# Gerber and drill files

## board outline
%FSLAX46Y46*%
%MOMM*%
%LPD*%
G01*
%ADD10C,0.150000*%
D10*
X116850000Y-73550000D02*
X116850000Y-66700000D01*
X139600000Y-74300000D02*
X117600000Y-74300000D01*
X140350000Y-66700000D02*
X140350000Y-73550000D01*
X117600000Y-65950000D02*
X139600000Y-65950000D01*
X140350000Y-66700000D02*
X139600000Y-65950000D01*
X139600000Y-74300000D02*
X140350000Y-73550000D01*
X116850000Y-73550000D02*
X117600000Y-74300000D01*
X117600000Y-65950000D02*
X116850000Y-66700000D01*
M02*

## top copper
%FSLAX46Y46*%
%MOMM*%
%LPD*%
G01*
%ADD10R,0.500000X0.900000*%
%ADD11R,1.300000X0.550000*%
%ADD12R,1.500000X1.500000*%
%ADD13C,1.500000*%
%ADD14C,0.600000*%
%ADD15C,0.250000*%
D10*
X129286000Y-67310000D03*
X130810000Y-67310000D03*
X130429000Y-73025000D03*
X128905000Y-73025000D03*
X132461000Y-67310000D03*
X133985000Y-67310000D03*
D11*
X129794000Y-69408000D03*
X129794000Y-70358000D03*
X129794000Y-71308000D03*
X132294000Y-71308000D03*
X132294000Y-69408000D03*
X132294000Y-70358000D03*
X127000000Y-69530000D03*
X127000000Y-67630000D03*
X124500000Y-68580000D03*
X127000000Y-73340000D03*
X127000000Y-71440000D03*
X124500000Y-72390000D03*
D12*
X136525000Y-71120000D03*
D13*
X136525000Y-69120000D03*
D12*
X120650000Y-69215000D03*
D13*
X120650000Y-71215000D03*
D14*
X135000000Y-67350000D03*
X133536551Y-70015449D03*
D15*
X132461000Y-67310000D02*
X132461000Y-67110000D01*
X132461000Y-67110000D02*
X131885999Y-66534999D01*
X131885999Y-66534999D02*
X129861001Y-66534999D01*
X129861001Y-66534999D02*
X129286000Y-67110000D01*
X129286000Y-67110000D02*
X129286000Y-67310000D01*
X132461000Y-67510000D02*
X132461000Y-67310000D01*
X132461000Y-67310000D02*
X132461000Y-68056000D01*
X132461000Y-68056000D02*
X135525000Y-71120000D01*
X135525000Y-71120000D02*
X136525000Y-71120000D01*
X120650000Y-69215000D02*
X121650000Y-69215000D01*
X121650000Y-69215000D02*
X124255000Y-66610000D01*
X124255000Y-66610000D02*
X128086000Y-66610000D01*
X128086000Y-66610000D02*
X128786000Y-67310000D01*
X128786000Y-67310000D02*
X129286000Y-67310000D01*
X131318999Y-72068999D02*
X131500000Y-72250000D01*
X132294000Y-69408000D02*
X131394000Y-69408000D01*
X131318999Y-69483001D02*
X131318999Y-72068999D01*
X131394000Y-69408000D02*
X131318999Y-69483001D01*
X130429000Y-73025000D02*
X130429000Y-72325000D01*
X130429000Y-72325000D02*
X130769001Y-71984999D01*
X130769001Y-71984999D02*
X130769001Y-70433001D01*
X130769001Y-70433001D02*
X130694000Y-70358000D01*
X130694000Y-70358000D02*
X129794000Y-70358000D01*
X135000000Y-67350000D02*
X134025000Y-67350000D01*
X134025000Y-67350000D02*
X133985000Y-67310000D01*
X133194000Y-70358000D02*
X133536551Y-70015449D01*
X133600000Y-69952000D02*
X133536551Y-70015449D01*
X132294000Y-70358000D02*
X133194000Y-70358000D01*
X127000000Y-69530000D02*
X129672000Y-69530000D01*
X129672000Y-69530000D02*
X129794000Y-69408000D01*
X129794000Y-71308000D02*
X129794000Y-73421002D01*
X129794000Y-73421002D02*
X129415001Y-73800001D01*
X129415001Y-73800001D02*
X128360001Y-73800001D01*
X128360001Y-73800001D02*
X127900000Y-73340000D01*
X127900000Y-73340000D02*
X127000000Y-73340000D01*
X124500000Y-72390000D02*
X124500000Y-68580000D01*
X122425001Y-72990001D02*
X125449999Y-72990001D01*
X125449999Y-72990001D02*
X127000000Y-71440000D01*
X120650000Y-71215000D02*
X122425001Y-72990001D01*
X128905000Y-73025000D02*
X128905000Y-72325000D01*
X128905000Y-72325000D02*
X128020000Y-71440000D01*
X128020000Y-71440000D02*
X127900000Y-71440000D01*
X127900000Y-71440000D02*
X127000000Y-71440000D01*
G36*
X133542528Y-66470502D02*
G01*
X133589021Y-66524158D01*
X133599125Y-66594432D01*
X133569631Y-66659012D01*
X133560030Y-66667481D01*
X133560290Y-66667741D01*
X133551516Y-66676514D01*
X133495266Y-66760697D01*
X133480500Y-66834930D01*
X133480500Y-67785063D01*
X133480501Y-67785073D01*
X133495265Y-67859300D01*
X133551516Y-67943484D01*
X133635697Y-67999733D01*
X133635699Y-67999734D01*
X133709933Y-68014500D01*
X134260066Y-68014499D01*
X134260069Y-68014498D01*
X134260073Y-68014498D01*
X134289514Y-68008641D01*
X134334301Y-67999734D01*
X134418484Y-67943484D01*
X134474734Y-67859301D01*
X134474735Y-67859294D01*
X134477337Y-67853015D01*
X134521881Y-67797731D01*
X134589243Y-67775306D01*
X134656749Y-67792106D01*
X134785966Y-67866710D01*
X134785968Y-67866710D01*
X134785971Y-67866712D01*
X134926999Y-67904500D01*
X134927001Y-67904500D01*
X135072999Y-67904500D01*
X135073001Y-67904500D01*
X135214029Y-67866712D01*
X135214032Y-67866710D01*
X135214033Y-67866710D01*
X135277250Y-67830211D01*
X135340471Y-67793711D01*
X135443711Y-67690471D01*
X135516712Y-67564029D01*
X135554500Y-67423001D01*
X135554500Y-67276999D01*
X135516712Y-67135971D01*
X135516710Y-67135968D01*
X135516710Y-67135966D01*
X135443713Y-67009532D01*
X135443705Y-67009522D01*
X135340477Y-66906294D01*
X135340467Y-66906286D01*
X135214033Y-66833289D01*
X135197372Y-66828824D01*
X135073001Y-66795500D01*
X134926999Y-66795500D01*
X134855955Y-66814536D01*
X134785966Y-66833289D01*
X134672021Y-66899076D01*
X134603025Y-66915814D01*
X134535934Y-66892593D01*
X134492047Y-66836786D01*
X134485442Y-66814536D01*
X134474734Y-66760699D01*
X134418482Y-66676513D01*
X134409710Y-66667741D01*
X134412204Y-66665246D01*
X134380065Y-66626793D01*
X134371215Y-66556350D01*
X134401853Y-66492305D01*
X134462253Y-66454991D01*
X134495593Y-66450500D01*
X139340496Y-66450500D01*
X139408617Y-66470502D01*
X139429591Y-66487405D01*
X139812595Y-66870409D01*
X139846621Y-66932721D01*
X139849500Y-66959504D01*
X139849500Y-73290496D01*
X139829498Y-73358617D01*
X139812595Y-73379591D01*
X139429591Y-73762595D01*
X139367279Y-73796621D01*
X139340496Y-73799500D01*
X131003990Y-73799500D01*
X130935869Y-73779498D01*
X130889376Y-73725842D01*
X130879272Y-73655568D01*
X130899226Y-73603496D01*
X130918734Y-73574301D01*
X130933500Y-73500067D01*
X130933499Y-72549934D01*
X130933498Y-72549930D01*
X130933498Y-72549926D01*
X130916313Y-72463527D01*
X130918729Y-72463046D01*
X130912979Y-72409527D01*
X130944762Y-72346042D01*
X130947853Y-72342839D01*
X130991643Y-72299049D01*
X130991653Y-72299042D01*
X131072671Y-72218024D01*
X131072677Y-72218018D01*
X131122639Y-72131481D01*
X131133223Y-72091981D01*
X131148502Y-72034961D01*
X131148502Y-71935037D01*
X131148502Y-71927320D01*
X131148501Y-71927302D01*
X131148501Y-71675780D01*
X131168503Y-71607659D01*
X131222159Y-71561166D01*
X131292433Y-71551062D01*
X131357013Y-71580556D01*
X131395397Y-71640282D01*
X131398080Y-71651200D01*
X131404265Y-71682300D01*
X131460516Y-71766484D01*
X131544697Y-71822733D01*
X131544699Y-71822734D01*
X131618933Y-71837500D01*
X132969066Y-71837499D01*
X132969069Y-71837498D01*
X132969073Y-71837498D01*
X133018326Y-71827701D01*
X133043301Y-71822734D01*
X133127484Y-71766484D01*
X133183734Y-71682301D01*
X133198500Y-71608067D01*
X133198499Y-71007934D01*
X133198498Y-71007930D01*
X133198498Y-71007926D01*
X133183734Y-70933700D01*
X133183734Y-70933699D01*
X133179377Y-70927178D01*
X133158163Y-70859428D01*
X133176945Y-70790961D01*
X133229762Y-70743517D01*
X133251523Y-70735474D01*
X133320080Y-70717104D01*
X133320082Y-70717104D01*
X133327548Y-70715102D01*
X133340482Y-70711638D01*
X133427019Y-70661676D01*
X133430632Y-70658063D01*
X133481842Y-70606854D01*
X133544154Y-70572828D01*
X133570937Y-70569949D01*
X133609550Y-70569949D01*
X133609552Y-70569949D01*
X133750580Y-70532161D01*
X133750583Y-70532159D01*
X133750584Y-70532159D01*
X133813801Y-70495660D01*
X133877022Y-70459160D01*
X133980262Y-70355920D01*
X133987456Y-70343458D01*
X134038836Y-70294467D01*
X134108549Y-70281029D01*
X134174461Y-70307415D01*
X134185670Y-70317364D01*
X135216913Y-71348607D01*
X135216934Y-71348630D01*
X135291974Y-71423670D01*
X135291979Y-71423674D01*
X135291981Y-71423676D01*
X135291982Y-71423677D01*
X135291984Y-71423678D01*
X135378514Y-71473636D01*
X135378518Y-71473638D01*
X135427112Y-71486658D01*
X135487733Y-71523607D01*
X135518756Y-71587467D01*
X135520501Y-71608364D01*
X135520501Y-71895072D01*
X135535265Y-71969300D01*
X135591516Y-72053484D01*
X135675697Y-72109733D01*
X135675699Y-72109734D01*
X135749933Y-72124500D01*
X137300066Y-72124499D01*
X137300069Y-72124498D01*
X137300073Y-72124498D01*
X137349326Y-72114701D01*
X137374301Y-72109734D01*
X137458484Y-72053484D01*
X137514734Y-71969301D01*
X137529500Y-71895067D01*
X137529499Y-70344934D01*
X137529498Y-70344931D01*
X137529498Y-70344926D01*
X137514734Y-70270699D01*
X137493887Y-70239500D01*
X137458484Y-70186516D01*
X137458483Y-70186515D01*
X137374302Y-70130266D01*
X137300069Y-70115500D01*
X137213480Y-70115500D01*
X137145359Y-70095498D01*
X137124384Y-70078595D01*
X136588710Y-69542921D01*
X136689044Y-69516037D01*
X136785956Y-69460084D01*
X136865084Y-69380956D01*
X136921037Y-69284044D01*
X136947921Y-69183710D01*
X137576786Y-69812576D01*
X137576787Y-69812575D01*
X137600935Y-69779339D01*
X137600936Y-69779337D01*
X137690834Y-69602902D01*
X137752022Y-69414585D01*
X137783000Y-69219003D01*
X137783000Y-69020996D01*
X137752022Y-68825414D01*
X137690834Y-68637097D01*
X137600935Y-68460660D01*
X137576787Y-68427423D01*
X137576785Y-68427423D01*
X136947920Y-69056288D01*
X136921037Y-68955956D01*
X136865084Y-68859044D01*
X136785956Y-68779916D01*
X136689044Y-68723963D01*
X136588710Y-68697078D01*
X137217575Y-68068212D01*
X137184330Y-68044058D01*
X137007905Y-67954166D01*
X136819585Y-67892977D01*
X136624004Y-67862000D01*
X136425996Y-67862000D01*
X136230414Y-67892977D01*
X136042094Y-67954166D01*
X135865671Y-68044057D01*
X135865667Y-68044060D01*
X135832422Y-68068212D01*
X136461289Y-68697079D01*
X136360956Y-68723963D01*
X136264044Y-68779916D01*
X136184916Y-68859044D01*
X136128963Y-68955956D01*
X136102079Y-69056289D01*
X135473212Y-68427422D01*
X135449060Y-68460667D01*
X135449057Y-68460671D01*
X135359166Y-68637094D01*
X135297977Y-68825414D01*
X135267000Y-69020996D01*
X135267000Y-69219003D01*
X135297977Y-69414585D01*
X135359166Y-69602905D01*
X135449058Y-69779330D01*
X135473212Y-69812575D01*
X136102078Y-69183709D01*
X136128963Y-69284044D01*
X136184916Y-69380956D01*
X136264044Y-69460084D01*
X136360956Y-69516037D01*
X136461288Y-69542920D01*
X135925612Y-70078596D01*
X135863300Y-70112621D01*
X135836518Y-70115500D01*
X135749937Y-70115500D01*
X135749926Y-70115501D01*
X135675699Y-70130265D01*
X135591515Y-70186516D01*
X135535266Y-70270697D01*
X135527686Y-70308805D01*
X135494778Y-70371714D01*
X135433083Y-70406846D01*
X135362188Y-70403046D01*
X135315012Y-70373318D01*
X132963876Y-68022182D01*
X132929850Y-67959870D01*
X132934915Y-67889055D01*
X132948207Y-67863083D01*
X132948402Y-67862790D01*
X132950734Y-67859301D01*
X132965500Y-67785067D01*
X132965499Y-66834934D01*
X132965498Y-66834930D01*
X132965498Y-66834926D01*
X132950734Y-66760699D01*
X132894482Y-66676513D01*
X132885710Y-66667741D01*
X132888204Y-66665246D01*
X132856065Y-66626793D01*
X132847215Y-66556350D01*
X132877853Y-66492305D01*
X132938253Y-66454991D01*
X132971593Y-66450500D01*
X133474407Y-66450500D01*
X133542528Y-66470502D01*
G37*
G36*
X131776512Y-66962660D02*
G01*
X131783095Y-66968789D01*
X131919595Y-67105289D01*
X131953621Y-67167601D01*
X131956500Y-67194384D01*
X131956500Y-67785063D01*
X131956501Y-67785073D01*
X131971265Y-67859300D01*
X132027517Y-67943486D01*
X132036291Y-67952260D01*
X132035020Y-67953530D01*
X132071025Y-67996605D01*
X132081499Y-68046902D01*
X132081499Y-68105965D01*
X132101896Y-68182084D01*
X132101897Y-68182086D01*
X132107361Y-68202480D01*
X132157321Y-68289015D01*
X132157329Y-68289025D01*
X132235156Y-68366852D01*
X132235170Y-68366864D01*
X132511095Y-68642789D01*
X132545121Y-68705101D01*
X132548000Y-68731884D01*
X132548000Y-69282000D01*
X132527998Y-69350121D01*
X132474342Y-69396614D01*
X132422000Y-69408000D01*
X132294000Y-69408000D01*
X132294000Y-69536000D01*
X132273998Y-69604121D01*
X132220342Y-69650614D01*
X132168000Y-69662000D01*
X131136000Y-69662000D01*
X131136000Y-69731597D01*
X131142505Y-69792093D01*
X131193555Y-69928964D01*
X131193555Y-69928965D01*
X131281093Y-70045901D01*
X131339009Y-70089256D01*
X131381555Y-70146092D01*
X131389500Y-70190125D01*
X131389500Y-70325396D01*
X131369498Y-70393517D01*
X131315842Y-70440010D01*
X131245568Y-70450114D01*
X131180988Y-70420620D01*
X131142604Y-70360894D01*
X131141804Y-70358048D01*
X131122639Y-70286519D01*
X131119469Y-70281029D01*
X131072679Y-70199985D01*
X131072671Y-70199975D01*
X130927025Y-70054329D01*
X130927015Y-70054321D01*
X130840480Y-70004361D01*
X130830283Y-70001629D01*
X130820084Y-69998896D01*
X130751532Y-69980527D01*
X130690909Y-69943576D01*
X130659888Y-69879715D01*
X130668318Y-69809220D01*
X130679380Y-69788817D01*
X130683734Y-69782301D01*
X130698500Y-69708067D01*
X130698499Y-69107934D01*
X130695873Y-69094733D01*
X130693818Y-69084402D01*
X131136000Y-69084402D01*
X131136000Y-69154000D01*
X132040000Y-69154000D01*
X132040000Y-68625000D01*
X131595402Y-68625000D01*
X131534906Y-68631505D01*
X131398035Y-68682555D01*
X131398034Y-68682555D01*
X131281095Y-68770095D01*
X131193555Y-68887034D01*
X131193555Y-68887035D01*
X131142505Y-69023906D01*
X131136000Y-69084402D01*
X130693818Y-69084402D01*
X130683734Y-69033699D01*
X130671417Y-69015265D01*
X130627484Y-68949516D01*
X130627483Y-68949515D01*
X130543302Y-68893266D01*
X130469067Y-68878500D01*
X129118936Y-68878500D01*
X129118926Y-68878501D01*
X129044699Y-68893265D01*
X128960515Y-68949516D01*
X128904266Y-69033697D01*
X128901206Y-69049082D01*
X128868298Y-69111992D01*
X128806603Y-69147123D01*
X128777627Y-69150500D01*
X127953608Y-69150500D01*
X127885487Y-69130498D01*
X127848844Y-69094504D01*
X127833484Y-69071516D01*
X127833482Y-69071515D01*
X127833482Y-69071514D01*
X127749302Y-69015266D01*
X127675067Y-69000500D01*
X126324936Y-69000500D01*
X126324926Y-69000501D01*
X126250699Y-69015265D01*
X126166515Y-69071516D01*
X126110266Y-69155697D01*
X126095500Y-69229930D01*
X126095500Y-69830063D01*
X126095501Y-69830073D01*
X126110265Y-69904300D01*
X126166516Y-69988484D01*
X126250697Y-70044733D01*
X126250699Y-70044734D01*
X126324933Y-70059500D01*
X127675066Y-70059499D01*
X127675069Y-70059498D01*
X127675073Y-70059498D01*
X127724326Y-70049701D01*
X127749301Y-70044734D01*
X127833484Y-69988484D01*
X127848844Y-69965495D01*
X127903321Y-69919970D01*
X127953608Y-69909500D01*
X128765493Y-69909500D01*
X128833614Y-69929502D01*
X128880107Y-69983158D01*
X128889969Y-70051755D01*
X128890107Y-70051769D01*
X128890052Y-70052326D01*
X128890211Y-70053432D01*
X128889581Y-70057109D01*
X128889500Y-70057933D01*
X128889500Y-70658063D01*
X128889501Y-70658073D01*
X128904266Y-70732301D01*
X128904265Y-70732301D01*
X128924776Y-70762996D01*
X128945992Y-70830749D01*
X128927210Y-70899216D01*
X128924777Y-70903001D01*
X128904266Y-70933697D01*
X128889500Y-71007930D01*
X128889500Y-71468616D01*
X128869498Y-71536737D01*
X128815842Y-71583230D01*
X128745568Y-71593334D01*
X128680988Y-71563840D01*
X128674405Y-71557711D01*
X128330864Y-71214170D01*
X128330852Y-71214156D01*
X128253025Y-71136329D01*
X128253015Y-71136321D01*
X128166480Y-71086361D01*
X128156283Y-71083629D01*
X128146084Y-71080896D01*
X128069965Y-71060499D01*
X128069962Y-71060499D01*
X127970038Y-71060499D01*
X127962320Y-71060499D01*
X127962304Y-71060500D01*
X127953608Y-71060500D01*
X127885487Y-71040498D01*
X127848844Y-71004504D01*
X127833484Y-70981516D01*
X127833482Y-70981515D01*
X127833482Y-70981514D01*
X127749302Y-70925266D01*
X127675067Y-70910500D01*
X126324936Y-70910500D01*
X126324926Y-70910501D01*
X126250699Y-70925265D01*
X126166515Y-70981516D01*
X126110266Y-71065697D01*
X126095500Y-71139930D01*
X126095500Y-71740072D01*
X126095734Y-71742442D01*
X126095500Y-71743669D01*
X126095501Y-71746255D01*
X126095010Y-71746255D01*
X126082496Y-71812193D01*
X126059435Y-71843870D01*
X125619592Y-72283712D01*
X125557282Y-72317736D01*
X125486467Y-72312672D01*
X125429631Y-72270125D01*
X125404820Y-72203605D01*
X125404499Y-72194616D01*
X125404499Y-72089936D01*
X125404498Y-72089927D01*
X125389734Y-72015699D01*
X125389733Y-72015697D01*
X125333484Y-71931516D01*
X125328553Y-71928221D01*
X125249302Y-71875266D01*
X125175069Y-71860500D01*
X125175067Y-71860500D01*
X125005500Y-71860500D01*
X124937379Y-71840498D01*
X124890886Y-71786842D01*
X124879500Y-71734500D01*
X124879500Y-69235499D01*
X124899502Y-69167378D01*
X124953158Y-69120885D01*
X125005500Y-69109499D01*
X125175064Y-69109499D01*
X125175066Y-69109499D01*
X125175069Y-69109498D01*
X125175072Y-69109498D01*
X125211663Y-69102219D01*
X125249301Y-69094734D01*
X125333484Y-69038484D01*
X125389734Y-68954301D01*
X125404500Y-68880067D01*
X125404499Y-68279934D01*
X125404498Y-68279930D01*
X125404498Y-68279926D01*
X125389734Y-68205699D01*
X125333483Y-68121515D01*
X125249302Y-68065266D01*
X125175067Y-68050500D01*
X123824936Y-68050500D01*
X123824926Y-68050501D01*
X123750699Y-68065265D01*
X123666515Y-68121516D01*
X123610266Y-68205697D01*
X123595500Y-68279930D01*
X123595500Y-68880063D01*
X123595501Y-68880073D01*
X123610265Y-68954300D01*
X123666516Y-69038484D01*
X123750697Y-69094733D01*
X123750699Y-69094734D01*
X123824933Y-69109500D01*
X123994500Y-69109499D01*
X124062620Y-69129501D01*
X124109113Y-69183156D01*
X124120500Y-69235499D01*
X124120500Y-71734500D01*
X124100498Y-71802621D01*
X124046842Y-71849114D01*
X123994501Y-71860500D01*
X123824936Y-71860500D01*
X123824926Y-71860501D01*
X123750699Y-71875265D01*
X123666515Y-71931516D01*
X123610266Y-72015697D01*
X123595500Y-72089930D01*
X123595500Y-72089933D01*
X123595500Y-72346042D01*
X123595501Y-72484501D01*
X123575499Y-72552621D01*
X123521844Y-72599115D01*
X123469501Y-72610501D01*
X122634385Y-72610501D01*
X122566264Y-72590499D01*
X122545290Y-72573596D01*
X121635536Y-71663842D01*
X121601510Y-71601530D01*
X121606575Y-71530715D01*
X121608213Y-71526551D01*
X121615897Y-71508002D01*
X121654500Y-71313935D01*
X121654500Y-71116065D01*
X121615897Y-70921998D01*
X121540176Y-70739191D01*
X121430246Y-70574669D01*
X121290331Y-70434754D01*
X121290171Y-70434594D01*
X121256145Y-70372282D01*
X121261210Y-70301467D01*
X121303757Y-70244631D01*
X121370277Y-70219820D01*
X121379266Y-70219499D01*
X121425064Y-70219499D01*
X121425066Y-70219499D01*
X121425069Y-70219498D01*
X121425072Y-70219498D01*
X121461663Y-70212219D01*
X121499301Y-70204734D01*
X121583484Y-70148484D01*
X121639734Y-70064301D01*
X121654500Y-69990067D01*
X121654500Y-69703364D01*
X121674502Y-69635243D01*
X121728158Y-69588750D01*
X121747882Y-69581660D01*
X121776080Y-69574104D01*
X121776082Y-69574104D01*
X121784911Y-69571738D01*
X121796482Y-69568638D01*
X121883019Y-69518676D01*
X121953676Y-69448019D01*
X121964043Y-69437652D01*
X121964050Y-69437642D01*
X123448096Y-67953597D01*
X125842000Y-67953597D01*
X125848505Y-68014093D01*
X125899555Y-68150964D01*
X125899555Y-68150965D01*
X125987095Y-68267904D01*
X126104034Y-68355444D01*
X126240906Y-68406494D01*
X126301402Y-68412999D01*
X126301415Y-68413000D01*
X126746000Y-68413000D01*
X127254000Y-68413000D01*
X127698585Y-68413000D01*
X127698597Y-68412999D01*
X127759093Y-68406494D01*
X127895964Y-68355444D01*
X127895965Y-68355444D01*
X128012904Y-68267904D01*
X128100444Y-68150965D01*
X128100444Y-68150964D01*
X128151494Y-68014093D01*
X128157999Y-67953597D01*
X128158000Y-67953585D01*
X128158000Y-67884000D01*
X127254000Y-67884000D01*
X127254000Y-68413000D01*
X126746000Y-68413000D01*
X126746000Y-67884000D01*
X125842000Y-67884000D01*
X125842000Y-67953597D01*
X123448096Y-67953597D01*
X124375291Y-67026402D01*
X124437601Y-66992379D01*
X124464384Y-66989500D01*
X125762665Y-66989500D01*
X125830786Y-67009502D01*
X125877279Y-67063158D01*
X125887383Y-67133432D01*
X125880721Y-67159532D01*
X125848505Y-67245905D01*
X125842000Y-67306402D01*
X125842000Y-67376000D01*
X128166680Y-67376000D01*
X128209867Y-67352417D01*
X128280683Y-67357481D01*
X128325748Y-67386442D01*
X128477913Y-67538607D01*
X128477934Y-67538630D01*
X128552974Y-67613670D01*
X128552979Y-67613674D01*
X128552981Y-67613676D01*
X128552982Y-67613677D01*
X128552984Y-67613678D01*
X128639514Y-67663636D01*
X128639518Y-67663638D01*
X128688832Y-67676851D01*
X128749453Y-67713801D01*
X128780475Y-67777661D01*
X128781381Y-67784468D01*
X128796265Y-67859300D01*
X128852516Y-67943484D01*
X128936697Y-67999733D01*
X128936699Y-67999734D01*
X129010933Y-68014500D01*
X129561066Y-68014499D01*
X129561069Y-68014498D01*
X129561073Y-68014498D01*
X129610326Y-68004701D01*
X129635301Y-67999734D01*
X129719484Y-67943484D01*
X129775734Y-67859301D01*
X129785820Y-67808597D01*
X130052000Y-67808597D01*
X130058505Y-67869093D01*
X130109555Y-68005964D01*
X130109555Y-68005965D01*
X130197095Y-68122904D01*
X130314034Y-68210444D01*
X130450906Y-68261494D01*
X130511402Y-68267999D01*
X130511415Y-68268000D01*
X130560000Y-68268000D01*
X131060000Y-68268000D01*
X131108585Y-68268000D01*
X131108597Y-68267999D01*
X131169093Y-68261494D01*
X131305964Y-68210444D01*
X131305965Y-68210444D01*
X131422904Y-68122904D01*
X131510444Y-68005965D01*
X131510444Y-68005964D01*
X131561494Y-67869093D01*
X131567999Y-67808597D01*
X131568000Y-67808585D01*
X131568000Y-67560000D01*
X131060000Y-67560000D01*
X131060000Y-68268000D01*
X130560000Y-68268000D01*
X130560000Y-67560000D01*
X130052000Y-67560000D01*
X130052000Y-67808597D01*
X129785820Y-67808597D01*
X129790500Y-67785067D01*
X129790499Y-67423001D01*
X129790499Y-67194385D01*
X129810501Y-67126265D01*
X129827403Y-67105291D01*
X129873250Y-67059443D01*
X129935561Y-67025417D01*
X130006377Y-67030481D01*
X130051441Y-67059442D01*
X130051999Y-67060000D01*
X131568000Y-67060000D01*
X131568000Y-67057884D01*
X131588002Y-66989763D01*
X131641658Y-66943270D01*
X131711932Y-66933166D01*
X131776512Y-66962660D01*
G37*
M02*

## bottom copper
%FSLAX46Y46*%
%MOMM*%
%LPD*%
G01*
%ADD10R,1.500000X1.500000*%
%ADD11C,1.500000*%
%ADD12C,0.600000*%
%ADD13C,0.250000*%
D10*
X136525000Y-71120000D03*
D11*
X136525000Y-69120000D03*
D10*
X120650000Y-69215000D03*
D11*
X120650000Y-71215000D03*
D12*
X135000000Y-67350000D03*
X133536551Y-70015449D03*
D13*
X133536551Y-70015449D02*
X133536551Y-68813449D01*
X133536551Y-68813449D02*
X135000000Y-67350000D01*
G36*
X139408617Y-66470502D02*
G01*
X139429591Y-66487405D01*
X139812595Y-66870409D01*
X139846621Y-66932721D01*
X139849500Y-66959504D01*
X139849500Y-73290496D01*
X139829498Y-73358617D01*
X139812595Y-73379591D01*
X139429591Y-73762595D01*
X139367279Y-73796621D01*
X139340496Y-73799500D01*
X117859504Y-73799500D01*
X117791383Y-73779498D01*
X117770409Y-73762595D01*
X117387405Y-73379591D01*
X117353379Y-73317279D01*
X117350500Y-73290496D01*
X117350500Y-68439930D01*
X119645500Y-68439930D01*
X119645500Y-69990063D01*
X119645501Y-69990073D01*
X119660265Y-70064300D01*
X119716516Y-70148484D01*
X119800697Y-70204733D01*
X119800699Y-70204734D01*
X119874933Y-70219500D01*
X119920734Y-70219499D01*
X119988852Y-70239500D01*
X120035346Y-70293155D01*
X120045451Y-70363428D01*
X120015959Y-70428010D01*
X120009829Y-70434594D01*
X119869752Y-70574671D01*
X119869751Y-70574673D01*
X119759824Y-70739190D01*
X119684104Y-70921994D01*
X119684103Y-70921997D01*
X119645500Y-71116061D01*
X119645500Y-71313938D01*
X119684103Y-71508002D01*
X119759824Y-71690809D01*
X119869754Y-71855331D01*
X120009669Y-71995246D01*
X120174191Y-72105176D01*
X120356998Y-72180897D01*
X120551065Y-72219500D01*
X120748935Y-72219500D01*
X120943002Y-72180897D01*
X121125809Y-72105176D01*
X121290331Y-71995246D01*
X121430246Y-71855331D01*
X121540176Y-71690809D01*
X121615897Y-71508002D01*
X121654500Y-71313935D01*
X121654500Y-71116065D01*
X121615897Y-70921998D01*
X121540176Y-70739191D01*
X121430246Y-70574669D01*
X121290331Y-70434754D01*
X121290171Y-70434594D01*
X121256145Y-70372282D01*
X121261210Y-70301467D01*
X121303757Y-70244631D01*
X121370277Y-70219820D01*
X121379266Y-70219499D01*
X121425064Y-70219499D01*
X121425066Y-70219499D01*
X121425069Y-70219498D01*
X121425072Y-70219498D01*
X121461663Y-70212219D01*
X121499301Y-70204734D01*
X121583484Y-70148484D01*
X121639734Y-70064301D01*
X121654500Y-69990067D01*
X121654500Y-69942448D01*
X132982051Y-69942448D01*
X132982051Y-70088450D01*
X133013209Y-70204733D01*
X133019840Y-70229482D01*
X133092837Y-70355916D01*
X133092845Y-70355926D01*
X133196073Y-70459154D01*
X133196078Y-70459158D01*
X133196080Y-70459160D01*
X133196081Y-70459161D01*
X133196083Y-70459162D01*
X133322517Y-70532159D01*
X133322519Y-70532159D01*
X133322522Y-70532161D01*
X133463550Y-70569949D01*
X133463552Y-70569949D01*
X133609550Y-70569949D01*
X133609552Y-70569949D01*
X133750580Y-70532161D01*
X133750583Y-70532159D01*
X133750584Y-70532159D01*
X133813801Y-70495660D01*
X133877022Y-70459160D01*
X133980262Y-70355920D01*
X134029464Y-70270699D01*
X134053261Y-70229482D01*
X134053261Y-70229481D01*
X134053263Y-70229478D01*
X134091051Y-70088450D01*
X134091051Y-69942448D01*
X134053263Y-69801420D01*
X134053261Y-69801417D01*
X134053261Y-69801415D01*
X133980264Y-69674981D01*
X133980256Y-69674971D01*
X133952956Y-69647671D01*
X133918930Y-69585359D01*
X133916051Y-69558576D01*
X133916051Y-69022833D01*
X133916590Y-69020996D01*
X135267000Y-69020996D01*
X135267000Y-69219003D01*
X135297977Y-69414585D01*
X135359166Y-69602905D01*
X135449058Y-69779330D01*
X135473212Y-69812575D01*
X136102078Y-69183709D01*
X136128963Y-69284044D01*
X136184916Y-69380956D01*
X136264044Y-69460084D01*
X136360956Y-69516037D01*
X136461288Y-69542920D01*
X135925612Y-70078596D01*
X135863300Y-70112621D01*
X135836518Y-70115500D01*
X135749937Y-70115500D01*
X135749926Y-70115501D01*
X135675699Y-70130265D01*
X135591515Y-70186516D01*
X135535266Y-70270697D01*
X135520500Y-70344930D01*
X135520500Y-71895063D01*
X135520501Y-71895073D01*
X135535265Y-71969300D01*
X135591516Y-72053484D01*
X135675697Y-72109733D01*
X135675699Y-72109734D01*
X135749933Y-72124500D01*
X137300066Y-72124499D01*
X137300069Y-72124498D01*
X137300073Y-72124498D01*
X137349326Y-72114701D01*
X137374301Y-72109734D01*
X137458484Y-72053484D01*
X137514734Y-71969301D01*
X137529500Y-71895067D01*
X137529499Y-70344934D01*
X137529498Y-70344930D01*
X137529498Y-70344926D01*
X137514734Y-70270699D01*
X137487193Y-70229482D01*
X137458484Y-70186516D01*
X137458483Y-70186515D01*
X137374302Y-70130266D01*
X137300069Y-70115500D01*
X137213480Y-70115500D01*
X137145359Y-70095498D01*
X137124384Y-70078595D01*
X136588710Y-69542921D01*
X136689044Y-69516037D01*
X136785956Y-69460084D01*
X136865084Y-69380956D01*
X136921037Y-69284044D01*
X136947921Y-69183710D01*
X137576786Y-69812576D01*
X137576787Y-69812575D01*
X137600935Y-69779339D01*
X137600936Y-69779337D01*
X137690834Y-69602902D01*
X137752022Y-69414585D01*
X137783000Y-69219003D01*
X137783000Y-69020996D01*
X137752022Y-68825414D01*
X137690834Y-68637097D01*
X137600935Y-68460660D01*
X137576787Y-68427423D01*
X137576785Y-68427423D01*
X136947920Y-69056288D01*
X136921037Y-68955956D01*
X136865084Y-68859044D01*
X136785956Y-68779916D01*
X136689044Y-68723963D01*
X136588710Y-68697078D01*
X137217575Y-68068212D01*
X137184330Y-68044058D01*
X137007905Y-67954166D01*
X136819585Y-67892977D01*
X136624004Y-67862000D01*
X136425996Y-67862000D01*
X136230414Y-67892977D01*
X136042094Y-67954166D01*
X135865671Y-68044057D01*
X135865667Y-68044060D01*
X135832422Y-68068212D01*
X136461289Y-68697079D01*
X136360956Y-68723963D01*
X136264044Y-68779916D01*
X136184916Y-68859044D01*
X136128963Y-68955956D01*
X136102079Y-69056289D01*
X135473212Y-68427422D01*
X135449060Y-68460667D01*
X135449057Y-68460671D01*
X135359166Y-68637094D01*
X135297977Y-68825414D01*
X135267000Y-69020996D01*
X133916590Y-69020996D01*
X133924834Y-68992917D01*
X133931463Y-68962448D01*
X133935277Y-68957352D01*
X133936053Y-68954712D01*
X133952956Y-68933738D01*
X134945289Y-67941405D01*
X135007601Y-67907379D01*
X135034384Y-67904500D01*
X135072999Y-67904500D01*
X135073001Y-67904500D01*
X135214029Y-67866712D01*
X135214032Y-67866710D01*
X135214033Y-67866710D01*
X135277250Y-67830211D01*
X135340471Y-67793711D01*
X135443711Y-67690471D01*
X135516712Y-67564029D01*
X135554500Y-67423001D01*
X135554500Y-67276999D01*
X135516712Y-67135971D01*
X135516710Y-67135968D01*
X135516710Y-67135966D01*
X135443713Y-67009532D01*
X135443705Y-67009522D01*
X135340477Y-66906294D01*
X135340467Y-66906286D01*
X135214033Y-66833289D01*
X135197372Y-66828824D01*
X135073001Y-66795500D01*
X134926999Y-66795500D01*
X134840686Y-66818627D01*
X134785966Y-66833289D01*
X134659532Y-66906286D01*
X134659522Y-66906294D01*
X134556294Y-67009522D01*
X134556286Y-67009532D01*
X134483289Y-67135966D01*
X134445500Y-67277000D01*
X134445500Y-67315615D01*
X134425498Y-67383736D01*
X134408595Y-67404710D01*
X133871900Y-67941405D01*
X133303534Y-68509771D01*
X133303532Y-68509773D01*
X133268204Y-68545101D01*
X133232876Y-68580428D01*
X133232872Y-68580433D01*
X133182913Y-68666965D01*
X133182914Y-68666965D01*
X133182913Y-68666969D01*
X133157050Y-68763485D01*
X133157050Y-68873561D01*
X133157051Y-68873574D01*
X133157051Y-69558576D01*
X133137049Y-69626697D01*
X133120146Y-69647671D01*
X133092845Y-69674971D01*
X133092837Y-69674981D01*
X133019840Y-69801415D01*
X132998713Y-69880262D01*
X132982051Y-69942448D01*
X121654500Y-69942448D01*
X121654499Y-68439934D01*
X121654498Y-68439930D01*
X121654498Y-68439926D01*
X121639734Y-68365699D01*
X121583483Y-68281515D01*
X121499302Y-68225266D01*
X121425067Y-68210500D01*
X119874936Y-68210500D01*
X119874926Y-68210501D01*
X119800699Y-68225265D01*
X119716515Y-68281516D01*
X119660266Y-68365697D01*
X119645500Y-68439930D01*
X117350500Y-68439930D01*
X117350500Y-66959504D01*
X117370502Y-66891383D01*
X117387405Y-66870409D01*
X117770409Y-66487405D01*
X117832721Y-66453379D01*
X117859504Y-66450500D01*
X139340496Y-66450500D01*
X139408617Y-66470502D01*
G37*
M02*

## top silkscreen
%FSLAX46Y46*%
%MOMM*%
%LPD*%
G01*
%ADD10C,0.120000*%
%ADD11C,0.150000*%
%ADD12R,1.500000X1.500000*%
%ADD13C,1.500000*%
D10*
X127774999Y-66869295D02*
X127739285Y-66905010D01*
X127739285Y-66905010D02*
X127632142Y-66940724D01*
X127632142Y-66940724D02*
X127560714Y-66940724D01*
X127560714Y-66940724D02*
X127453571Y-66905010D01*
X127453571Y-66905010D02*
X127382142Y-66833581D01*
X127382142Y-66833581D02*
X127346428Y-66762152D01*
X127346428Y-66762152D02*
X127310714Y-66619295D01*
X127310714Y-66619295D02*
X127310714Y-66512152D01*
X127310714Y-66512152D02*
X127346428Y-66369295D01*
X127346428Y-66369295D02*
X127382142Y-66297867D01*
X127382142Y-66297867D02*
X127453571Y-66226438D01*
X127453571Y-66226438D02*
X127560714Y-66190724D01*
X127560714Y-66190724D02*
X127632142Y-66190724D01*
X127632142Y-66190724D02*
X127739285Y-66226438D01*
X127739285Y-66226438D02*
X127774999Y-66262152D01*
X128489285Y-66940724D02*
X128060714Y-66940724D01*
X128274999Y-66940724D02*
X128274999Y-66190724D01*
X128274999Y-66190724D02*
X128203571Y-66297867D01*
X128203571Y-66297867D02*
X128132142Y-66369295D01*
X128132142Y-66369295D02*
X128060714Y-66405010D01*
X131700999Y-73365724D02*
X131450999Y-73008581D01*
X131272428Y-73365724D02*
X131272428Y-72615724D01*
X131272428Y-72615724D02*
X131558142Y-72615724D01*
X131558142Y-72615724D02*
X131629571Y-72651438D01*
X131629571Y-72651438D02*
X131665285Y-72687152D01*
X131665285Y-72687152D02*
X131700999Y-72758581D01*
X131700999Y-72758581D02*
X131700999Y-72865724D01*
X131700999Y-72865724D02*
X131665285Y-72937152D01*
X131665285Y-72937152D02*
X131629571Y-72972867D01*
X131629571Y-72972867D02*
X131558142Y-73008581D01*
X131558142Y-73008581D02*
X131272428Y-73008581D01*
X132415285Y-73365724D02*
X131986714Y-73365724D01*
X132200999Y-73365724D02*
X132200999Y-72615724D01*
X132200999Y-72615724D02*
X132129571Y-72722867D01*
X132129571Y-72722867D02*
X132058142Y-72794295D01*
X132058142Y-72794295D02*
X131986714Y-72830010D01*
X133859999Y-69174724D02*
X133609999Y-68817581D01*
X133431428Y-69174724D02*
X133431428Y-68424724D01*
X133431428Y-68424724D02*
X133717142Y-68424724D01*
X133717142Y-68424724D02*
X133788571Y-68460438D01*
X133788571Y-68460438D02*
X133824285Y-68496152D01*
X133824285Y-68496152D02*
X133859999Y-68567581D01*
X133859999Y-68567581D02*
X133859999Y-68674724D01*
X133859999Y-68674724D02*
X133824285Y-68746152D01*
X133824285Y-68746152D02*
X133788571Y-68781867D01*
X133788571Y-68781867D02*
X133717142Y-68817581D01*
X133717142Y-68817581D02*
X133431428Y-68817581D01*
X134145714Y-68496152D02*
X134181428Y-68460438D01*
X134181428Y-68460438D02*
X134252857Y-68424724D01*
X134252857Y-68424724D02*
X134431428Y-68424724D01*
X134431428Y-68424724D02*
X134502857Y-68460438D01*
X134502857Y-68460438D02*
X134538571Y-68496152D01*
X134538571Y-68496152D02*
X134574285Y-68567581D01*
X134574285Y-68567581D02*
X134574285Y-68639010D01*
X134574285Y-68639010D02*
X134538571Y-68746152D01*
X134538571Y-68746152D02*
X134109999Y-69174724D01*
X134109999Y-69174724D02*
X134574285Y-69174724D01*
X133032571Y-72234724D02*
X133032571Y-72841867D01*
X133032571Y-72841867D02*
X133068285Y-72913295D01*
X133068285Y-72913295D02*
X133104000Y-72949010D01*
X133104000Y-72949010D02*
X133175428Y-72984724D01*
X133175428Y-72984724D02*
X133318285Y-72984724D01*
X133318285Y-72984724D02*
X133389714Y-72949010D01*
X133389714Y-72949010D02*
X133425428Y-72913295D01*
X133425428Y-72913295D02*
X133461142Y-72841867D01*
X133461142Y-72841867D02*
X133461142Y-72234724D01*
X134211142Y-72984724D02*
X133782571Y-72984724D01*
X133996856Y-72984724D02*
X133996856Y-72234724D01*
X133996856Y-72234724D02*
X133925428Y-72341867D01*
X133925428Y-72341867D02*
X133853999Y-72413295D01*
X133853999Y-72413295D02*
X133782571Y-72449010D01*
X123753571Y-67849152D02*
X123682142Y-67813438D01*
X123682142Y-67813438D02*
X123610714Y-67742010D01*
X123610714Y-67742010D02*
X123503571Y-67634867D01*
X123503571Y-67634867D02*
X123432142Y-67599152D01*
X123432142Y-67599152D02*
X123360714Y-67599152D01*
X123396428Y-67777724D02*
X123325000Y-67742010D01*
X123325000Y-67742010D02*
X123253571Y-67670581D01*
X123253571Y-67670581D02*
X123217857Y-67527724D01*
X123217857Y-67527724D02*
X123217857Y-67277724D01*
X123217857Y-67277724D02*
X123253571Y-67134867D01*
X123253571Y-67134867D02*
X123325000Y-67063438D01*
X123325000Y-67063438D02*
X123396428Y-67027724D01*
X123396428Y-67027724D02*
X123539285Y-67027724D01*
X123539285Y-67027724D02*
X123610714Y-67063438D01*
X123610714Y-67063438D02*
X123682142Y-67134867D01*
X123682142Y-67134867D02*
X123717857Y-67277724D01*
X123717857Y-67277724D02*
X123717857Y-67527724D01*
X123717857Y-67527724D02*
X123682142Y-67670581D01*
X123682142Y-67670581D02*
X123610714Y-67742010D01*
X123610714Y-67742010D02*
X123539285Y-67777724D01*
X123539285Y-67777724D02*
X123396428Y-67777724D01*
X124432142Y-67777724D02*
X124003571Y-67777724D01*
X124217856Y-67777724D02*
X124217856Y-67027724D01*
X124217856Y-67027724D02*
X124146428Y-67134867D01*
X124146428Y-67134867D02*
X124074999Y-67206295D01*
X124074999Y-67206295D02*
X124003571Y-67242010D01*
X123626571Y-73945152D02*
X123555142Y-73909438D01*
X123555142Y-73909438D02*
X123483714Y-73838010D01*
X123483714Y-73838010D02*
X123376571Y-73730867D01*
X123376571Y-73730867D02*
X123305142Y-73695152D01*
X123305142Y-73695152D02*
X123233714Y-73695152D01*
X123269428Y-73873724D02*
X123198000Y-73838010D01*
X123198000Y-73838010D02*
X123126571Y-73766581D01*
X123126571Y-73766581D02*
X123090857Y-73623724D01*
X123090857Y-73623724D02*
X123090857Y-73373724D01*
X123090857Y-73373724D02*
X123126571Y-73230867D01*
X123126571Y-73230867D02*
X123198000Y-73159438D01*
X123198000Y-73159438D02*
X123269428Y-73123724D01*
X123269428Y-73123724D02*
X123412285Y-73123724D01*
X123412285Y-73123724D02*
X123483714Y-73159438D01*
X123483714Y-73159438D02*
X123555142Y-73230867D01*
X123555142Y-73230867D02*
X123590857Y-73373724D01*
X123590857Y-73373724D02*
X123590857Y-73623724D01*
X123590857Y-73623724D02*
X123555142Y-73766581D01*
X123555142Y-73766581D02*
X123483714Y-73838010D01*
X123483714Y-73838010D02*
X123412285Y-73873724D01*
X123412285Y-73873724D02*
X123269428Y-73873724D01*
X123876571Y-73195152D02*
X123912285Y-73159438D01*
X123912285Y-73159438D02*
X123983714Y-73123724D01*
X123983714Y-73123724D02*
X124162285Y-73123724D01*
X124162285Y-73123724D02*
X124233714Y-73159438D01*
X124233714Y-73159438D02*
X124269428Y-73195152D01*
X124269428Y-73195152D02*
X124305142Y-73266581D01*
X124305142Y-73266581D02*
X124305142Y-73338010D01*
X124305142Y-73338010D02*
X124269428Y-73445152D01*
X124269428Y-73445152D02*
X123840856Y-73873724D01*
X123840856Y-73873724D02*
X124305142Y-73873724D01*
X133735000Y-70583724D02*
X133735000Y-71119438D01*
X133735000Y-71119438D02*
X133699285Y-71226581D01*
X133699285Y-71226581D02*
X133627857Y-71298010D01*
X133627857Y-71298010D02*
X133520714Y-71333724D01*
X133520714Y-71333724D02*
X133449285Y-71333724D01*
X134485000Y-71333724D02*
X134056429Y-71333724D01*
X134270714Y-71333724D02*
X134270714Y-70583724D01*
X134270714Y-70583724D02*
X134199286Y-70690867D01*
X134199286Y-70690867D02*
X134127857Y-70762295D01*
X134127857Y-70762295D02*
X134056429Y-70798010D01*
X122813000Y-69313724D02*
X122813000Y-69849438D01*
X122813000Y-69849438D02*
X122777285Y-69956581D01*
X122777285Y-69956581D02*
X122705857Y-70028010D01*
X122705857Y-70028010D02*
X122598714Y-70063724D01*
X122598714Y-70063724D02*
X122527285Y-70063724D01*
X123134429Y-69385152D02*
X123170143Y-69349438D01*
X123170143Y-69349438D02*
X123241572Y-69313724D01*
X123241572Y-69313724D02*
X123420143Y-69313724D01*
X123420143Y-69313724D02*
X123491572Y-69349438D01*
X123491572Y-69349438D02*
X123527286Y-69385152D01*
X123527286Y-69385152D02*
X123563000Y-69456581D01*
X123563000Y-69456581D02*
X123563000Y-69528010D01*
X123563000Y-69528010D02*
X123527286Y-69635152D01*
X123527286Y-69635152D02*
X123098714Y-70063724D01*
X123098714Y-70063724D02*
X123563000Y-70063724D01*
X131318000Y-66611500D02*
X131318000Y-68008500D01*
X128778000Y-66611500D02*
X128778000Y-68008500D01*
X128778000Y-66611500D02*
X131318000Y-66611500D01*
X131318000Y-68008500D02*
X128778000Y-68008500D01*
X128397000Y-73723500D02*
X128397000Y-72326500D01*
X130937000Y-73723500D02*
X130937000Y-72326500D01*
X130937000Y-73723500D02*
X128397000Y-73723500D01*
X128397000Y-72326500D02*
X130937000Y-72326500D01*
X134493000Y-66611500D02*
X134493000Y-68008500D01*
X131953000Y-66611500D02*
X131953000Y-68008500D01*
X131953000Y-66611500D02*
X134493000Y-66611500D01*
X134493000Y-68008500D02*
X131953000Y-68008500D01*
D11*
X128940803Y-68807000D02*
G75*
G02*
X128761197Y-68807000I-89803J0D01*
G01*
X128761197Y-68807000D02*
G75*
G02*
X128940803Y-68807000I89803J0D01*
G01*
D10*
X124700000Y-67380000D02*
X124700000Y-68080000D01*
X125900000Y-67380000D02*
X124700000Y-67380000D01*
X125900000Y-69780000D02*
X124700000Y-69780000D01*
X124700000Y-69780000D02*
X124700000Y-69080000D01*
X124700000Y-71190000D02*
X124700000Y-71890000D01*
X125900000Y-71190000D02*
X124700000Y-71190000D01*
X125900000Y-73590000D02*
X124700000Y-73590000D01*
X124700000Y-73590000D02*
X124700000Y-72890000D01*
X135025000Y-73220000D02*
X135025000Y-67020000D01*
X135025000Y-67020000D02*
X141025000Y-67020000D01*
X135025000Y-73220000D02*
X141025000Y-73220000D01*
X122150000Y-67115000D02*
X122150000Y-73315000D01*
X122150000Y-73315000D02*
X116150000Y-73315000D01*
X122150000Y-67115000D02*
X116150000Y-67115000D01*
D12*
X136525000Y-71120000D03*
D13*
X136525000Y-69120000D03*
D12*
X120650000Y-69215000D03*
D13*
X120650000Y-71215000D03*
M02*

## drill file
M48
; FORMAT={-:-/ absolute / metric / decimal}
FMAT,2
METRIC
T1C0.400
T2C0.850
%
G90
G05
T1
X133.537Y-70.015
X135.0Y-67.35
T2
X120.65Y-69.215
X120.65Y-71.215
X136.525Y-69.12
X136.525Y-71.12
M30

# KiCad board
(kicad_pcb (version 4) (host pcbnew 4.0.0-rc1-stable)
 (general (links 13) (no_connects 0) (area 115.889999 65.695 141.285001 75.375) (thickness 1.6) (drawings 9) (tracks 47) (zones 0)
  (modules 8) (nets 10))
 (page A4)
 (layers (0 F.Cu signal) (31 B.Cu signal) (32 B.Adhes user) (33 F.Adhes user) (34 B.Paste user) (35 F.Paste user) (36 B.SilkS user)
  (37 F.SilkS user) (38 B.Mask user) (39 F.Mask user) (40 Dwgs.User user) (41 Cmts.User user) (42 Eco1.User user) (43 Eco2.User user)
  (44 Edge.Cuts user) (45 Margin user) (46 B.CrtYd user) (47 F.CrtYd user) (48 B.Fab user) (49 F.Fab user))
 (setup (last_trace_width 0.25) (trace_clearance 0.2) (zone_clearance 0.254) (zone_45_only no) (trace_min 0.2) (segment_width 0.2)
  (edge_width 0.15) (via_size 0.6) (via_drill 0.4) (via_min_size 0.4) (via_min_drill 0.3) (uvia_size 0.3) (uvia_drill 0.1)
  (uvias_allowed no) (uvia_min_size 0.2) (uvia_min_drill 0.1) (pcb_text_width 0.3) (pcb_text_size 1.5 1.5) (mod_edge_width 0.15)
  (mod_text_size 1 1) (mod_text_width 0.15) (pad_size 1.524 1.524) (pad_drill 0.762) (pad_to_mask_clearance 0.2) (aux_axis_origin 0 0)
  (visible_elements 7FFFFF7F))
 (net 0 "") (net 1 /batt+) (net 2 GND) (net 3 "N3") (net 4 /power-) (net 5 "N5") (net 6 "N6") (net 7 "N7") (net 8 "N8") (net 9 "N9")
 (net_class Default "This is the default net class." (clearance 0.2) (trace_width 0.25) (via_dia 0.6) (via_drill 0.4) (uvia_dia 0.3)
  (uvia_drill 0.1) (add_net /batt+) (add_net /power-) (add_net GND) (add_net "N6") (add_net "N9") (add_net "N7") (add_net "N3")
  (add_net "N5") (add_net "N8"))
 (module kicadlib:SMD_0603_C (layer F.Cu) (at 130.81 67.31)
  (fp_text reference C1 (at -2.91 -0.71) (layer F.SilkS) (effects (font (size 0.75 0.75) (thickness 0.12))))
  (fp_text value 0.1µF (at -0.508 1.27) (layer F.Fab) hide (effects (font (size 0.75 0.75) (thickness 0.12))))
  (fp_line (start 0.508 -0.6985) (end 0.508 0.6985) (layer F.SilkS) (width 0.12))
  (fp_line (start -2.032 -0.6985) (end -2.032 0.6985) (layer F.SilkS) (width 0.12))
  (fp_line (start -2.032 -0.6985) (end 0.508 -0.6985) (layer F.SilkS) (width 0.12))
  (fp_line (start 0.508 0.6985) (end -2.032 0.6985) (layer F.SilkS) (width 0.12))
  (pad 1 smd rect (at -1.524 0) (size 0.5 0.9) (layers F.Cu F.Paste F.Mask) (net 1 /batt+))
  (pad 2 smd rect (at 0 0) (size 0.5 0.9) (layers F.Cu F.Paste F.Mask) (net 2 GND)))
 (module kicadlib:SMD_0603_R (layer F.Cu) (at 128.905 73.025 180)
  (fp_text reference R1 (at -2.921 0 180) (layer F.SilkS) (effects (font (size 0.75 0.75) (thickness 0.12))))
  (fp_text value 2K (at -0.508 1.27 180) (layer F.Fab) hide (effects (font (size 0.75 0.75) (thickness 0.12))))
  (fp_line (start 0.508 -0.6985) (end 0.508 0.6985) (layer F.SilkS) (width 0.12))
  (fp_line (start -2.032 -0.6985) (end -2.032 0.6985) (layer F.SilkS) (width 0.12))
  (fp_line (start -2.032 -0.6985) (end 0.508 -0.6985) (layer F.SilkS) (width 0.12))
  (fp_line (start 0.508 0.6985) (end -2.032 0.6985) (layer F.SilkS) (width 0.12))
  (pad 1 smd rect (at -1.524 0 180) (size 0.5 0.9) (layers F.Cu F.Paste F.Mask) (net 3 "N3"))
  (pad 2 smd rect (at 0 0 180) (size 0.5 0.9) (layers F.Cu F.Paste F.Mask) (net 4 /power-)))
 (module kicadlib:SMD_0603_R (layer F.Cu) (at 133.985 67.31)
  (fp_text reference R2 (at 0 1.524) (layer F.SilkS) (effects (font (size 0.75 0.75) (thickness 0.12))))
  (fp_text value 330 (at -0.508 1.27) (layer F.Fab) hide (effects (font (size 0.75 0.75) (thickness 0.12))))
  (fp_line (start 0.508 -0.6985) (end 0.508 0.6985) (layer F.SilkS) (width 0.12))
  (fp_line (start -2.032 -0.6985) (end -2.032 0.6985) (layer F.SilkS) (width 0.12))
  (fp_line (start -2.032 -0.6985) (end 0.508 -0.6985) (layer F.SilkS) (width 0.12))
  (fp_line (start 0.508 0.6985) (end -2.032 0.6985) (layer F.SilkS) (width 0.12))
  (pad 1 smd rect (at -1.524 0) (size 0.5 0.9) (layers F.Cu F.Paste F.Mask) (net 1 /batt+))
  (pad 2 smd rect (at 0 0) (size 0.5 0.9) (layers F.Cu F.Paste F.Mask) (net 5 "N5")))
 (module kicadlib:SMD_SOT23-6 (layer F.Cu) (at 129.794 70.358)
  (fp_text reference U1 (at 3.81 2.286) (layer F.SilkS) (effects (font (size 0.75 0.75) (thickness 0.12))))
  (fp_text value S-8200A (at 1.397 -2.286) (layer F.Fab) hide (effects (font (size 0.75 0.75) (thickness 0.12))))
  (fp_circle (center -0.943 -1.551) (end -0.8795 -1.4875) (layer F.SilkS) (width 0.15))
  (pad 1 smd rect (at 0 -0.95) (size 1.3 0.55) (layers F.Cu F.Paste F.Mask) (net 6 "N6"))
  (pad 2 smd rect (at 0 0) (size 1.3 0.55) (layers F.Cu F.Paste F.Mask) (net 3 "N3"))
  (pad 3 smd rect (at 0 0.95) (size 1.3 0.55) (layers F.Cu F.Paste F.Mask) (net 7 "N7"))
  (pad 4 smd rect (at 2.5 0.95) (size 1.3 0.55) (layers F.Cu F.Paste F.Mask) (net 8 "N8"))
  (pad 6 smd rect (at 2.5 -0.95) (size 1.3 0.55) (layers F.Cu F.Paste F.Mask) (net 2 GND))
  (pad 5 smd rect (at 2.5 0) (size 1.3 0.55) (layers F.Cu F.Paste F.Mask) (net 5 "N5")))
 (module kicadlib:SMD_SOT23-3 (layer F.Cu) (at 127 68.58 180)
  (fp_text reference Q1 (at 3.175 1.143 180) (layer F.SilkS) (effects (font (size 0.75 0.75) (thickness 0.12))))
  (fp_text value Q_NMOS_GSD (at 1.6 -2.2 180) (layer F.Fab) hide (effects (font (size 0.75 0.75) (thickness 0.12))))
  (fp_line (start 2.3 1.2) (end 2.3 0.5) (layer F.SilkS) (width 0.12))
  (fp_line (start 1.1 1.2) (end 2.3 1.2) (layer F.SilkS) (width 0.12))
  (fp_line (start 1.1 -1.2) (end 2.3 -1.2) (layer F.SilkS) (width 0.12))
  (fp_line (start 2.3 -1.2) (end 2.3 -0.5) (layer F.SilkS) (width 0.12))
  (pad 1 smd rect (at 0 -0.95 180) (size 1.3 0.55) (layers F.Cu F.Paste F.Mask) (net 6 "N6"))
  (pad 2 smd rect (at 0 0.95 180) (size 1.3 0.55) (layers F.Cu F.Paste F.Mask) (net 2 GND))
  (pad 3 smd rect (at 2.5 0 180) (size 1.3 0.55) (layers F.Cu F.Paste F.Mask) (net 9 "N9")))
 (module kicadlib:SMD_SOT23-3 (layer F.Cu) (at 127 72.39 180)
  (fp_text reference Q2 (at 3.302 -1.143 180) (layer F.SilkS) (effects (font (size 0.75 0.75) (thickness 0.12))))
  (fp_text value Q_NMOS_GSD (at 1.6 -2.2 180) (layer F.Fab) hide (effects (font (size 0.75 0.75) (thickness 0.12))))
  (fp_line (start 2.3 1.2) (end 2.3 0.5) (layer F.SilkS) (width 0.12))
  (fp_line (start 1.1 1.2) (end 2.3 1.2) (layer F.SilkS) (width 0.12))
  (fp_line (start 1.1 -1.2) (end 2.3 -1.2) (layer F.SilkS) (width 0.12))
  (fp_line (start 2.3 -1.2) (end 2.3 -0.5) (layer F.SilkS) (width 0.12))
  (pad 1 smd rect (at 0 -0.95 180) (size 1.3 0.55) (layers F.Cu F.Paste F.Mask) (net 7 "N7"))
  (pad 2 smd rect (at 0 0.95 180) (size 1.3 0.55) (layers F.Cu F.Paste F.Mask) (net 4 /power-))
  (pad 3 smd rect (at 2.5 0 180) (size 1.3 0.55) (layers F.Cu F.Paste F.Mask) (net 9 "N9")))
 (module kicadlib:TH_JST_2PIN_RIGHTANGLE (layer F.Cu) (at 136.525 71.12 90)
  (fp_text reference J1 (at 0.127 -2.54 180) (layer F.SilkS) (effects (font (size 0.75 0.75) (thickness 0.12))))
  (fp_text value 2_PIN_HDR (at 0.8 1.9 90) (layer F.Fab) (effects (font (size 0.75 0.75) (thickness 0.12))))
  (fp_line (start -2.1 -1.5) (end 4.1 -1.5) (layer F.SilkS) (width 0.12))
  (fp_line (start 4.1 -1.5) (end 4.1 4.5) (layer F.SilkS) (width 0.12))
  (fp_line (start -2.1 -1.5) (end -2.1 4.5) (layer F.SilkS) (width 0.12))
  (pad 1 thru_hole rect (at 0 0 90) (size 1.5 1.5) (drill 0.85) (layers *.Cu *.Mask F.SilkS) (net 1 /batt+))
  (pad 2 thru_hole circle (at 2 0 90) (size 1.5 1.5) (drill 0.85) (layers *.Cu *.Mask F.SilkS) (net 2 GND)))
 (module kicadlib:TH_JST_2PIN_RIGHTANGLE (layer F.Cu) (at 120.65 69.215 270)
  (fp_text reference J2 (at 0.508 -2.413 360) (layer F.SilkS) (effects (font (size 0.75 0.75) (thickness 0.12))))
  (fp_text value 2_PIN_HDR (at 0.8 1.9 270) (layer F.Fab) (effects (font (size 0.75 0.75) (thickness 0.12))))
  (fp_line (start -2.1 -1.5) (end 4.1 -1.5) (layer F.SilkS) (width 0.12))
  (fp_line (start 4.1 -1.5) (end 4.1 4.5) (layer F.SilkS) (width 0.12))
  (fp_line (start -2.1 -1.5) (end -2.1 4.5) (layer F.SilkS) (width 0.12))
  (pad 1 thru_hole rect (at 0 0 270) (size 1.5 1.5) (drill 0.85) (layers *.Cu *.Mask F.SilkS) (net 1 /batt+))
  (pad 2 thru_hole circle (at 2 0 270) (size 1.5 1.5) (drill 0.85) (layers *.Cu *.Mask F.SilkS) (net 4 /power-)))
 (gr_line (start 116.85 73.55) (end 116.85 66.7) (angle 90) (layer Edge.Cuts) (width 0.15))
 (gr_line (start 139.6 74.3) (end 117.6 74.3) (angle 90) (layer Edge.Cuts) (width 0.15))
 (gr_line (start 140.35 66.7) (end 140.35 73.55) (angle 90) (layer Edge.Cuts) (width 0.15))
 (gr_line (start 117.6 65.95) (end 139.6 65.95) (angle 90) (layer Edge.Cuts) (width 0.15))
 (gr_line (start 140.35 66.7) (end 139.6 65.95) (angle 90) (layer Edge.Cuts) (width 0.15))
 (gr_line (start 139.6 74.3) (end 140.35 73.55) (angle 90) (layer Edge.Cuts) (width 0.15))
 (gr_line (start 116.85 73.55) (end 117.6 74.3) (angle 90) (layer Edge.Cuts) (width 0.15))
 (gr_line (start 117.6 65.95) (end 116.85 66.7) (angle 90) (layer Edge.Cuts) (width 0.15))
 (segment (start 132.461 67.31) (end 132.461 67.11) (width 0.25) (layer F.Cu) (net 1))
 (segment (start 132.461 67.11) (end 131.885999 66.534999) (width 0.25) (layer F.Cu) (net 1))
 (segment (start 131.885999 66.534999) (end 129.861001 66.534999) (width 0.25) (layer F.Cu) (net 1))
 (segment (start 129.861001 66.534999) (end 129.286 67.11) (width 0.25) (layer F.Cu) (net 1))
 (segment (start 129.286 67.11) (end 129.286 67.31) (width 0.25) (layer F.Cu) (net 1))
 (segment (start 132.461 67.51) (end 132.461 67.31) (width 0.25) (layer F.Cu) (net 1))
 (segment (start 132.461 67.31) (end 132.461 68.056) (width 0.25) (layer F.Cu) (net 1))
 (segment (start 132.461 68.056) (end 135.525 71.12) (width 0.25) (layer F.Cu) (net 1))
 (segment (start 135.525 71.12) (end 136.525 71.12) (width 0.25) (layer F.Cu) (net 1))
 (segment (start 120.65 69.215) (end 121.65 69.215) (width 0.25) (layer F.Cu) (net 1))
 (segment (start 121.65 69.215) (end 124.255 66.61) (width 0.25) (layer F.Cu) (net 1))
 (segment (start 124.255 66.61) (end 128.086 66.61) (width 0.25) (layer F.Cu) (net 1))
 (segment (start 128.086 66.61) (end 128.786 67.31) (width 0.25) (layer F.Cu) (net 1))
 (segment (start 128.786 67.31) (end 129.286 67.31) (width 0.25) (layer F.Cu) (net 1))
 (segment (start 131.318999 72.068999) (end 131.5 72.25) (width 0.25) (layer F.Cu) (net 2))
 (segment (start 132.294 69.408) (end 131.394 69.408) (width 0.25) (layer F.Cu) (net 2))
 (segment (start 131.318999 69.483001) (end 131.318999 72.068999) (width 0.25) (layer F.Cu) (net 2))
 (segment (start 131.394 69.408) (end 131.318999 69.483001) (width 0.25) (layer F.Cu) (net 2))
 (segment (start 130.429 73.025) (end 130.429 72.325) (width 0.25) (layer F.Cu) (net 3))
 (segment (start 130.429 72.325) (end 130.769001 71.984999) (width 0.25) (layer F.Cu) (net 3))
 (segment (start 130.769001 71.984999) (end 130.769001 70.433001) (width 0.25) (layer F.Cu) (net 3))
 (segment (start 130.769001 70.433001) (end 130.694 70.358) (width 0.25) (layer F.Cu) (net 3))
 (segment (start 130.694 70.358) (end 129.794 70.358) (width 0.25) (layer F.Cu) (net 3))
 (segment (start 135 67.35) (end 134.025 67.35) (width 0.25) (layer F.Cu) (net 5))
 (segment (start 134.025 67.35) (end 133.985 67.31) (width 0.25) (layer F.Cu) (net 5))
 (segment (start 133.536551 70.015449) (end 133.536551 68.813449) (width 0.25) (layer B.Cu) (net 5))
 (via (at 135 67.35) (size 0.6) (drill 0.4) (layers F.Cu B.Cu) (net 5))
 (segment (start 133.536551 68.813449) (end 135 67.35) (width 0.25) (layer B.Cu) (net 5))
 (segment (start 133.194 70.358) (end 133.536551 70.015449) (width 0.25) (layer F.Cu) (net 5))
 (segment (start 133.6 69.952) (end 133.536551 70.015449) (width 0.25) (layer F.Cu) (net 5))
 (via (at 133.536551 70.015449) (size 0.6) (drill 0.4) (layers F.Cu B.Cu) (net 5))
 (segment (start 132.294 70.358) (end 133.194 70.358) (width 0.25) (layer F.Cu) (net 5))
 (segment (start 127 69.53) (end 129.672 69.53) (width 0.25) (layer F.Cu) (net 6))
 (segment (start 129.672 69.53) (end 129.794 69.408) (width 0.25) (layer F.Cu) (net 6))
 (segment (start 129.794 71.308) (end 129.794 73.421002) (width 0.25) (layer F.Cu) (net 7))
 (segment (start 129.794 73.421002) (end 129.415001 73.800001) (width 0.25) (layer F.Cu) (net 7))
 (segment (start 129.415001 73.800001) (end 128.360001 73.800001) (width 0.25) (layer F.Cu) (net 7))
 (segment (start 128.360001 73.800001) (end 127.9 73.34) (width 0.25) (layer F.Cu) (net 7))
 (segment (start 127.9 73.34) (end 127 73.34) (width 0.25) (layer F.Cu) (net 7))
 (segment (start 124.5 72.39) (end 124.5 68.58) (width 0.25) (layer F.Cu) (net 9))
 (segment (start 122.425001 72.990001) (end 125.449999 72.990001) (width 0.25) (layer F.Cu) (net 4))
 (segment (start 125.449999 72.990001) (end 127 71.44) (width 0.25) (layer F.Cu) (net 4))
 (segment (start 120.65 71.215) (end 122.425001 72.990001) (width 0.25) (layer F.Cu) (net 4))
 (segment (start 128.905 73.025) (end 128.905 72.325) (width 0.25) (layer F.Cu) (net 4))
 (segment (start 128.905 72.325) (end 128.02 71.44) (width 0.25) (layer F.Cu) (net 4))
 (segment (start 128.02 71.44) (end 127.9 71.44) (width 0.25) (layer F.Cu) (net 4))
 (segment (start 127.9 71.44) (end 127 71.44) (width 0.25) (layer F.Cu) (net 4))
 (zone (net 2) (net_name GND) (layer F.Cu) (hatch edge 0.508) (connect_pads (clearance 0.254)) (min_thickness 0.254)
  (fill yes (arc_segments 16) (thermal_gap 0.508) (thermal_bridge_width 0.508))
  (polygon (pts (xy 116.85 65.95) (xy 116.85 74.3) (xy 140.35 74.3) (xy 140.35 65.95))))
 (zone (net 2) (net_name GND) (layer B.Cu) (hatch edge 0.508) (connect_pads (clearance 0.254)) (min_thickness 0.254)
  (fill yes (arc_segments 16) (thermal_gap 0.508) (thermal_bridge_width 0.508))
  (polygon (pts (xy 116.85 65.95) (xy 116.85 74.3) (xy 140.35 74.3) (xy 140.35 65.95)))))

